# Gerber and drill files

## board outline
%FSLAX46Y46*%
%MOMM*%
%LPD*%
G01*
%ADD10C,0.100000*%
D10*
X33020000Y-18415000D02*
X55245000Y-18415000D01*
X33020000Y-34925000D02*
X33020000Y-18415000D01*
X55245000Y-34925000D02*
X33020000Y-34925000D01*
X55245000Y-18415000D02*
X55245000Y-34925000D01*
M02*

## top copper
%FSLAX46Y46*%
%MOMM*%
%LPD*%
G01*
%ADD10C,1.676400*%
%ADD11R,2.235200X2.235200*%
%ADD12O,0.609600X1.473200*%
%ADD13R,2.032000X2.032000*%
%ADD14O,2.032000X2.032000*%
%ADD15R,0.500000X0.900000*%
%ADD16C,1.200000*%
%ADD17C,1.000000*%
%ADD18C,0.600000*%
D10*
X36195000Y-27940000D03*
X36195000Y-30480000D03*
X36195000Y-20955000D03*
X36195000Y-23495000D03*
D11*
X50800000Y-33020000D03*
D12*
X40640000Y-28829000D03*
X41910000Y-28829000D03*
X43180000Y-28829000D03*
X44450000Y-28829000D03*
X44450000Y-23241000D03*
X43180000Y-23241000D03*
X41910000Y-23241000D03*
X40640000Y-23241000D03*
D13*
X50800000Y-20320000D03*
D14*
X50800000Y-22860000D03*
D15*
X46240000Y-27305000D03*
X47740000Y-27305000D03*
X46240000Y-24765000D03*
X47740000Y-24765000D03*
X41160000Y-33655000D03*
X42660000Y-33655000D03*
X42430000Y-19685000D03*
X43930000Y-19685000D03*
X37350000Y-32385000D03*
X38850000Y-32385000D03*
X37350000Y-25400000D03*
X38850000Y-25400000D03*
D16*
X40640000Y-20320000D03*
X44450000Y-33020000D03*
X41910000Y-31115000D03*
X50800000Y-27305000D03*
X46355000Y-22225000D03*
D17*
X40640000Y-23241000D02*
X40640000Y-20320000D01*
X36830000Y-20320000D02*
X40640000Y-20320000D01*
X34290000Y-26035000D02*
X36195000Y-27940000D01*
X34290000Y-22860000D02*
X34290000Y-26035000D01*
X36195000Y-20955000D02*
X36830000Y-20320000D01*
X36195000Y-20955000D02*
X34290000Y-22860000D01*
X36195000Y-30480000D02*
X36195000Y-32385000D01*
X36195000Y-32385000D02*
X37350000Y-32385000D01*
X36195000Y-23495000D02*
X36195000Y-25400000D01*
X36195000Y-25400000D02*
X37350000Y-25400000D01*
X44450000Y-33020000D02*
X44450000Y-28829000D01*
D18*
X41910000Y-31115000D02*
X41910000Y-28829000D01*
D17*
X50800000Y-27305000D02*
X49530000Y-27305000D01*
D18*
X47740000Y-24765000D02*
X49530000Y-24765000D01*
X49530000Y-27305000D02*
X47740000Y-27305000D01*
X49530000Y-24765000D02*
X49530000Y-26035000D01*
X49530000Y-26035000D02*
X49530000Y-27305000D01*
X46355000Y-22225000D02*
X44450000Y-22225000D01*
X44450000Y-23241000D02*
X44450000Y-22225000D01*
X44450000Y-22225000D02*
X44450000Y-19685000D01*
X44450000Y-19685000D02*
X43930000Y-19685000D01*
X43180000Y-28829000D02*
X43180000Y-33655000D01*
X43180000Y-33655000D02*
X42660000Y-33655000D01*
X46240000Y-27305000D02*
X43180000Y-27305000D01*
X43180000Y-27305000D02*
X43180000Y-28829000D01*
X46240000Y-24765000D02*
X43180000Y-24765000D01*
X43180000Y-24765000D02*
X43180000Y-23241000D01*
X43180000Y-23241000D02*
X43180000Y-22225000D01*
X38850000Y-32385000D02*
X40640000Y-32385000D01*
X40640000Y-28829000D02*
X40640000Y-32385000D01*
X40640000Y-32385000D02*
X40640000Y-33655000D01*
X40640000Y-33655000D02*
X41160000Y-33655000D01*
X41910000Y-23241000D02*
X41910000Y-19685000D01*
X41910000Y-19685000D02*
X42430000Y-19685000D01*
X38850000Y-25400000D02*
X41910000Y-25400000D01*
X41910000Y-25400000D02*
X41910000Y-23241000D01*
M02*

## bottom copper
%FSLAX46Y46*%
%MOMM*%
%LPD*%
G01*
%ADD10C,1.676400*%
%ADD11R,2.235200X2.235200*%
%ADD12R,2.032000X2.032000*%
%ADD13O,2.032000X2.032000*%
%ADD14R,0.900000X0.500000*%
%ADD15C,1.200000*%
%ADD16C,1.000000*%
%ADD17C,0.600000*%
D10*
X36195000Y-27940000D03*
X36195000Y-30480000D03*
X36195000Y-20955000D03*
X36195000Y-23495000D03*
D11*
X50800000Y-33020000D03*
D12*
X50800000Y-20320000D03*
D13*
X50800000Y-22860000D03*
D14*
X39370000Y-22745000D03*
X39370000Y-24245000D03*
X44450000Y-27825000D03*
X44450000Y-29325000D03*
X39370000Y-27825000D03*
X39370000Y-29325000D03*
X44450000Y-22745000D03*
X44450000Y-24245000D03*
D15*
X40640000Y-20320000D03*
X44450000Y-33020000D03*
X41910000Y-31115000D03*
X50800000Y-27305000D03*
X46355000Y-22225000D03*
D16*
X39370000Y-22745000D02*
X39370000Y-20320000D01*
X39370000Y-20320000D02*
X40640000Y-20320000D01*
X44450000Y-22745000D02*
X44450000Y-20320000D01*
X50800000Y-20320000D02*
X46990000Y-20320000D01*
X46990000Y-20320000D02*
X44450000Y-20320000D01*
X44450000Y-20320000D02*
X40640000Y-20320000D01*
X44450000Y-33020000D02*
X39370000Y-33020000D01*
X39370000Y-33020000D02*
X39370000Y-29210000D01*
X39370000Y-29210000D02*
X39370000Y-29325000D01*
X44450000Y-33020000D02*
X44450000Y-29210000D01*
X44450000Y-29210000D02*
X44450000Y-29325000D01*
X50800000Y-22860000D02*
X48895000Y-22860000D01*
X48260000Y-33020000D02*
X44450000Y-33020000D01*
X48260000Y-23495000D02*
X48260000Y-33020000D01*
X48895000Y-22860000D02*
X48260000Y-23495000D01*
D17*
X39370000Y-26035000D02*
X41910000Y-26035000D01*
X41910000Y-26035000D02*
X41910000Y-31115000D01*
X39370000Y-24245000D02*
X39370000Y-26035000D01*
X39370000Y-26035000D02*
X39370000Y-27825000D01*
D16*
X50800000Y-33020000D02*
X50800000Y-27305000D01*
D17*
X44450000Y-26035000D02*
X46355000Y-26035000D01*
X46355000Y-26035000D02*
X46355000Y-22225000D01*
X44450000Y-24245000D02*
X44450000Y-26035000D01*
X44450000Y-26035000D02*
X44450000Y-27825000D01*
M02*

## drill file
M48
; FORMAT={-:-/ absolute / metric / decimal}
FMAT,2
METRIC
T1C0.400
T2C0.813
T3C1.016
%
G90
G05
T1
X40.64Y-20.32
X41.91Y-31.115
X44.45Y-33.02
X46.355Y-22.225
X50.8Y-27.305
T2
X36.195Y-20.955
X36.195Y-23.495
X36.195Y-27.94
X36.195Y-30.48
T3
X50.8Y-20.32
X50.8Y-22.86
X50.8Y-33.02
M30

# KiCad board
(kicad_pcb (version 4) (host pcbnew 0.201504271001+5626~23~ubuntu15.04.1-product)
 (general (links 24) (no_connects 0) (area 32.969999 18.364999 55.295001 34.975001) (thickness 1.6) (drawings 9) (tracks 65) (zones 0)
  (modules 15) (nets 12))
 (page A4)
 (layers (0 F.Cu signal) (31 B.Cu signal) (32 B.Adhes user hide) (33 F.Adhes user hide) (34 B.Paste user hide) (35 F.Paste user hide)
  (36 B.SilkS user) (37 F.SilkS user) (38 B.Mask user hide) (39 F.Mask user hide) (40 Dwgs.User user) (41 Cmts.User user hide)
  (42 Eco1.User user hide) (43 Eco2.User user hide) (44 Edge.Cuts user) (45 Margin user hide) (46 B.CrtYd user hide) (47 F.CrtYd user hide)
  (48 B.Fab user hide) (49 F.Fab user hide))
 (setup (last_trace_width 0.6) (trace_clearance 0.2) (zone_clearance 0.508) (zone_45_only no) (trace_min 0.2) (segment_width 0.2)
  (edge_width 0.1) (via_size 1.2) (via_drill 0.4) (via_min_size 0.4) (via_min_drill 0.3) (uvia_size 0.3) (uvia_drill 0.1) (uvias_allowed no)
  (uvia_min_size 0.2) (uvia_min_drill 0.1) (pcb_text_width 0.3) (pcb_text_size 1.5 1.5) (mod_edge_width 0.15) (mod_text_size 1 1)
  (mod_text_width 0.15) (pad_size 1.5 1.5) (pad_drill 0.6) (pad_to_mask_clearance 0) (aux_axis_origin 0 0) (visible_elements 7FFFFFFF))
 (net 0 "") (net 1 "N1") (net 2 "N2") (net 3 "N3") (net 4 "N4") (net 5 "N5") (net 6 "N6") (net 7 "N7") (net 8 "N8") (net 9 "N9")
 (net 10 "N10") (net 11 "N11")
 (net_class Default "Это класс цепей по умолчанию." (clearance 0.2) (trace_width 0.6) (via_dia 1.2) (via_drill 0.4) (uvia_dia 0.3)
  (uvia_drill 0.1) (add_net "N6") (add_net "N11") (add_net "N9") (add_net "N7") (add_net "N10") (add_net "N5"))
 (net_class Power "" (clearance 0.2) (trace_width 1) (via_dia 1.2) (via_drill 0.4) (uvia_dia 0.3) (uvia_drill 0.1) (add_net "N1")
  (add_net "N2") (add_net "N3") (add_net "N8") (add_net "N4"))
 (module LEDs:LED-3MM (layer B.Cu) (at 36.195 29.21 270)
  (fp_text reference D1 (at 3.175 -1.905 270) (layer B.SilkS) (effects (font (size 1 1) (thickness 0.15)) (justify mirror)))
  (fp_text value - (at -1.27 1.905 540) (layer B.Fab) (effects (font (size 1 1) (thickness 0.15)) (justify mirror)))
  (pad 1 thru_hole circle (at -1.27 0 270) (size 1.6764 1.6764) (drill 0.8128) (layers *.Cu *.Mask B.SilkS) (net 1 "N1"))
  (pad 2 thru_hole circle (at 1.27 0 270) (size 1.6764 1.6764) (drill 0.8128) (layers *.Cu *.Mask B.SilkS) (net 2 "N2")))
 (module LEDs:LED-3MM (layer B.Cu) (at 36.195 22.225 270)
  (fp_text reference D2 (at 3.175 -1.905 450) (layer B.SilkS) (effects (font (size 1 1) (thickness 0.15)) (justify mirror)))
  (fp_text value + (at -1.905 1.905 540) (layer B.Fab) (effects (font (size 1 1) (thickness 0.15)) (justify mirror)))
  (pad 1 thru_hole circle (at -1.27 0 270) (size 1.6764 1.6764) (drill 0.8128) (layers *.Cu *.Mask B.SilkS) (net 1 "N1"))
  (pad 2 thru_hole circle (at 1.27 0 270) (size 1.6764 1.6764) (drill 0.8128) (layers *.Cu *.Mask B.SilkS) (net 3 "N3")))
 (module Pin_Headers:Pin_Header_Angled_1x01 (layer F.Cu) (at 50.8 33.02)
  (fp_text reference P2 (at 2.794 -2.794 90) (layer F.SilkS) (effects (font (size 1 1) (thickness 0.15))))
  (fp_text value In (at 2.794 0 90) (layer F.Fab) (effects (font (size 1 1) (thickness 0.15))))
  (pad 1 thru_hole rect (at 0 0) (size 2.2352 2.2352) (drill 1.016) (layers *.Cu *.Mask F.SilkS) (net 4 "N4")))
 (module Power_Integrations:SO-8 (layer F.Cu) (at 42.545 26.035)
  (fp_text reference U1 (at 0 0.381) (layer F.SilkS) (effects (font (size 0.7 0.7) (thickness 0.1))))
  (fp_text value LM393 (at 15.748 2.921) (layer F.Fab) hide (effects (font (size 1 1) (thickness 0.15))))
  (pad 1 smd oval (at -1.905 2.794) (size 0.6096 1.4732) (layers F.Cu F.Paste F.Mask) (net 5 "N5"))
  (pad 2 smd oval (at -0.635 2.794) (size 0.6096 1.4732) (layers F.Cu F.Paste F.Mask) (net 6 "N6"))
  (pad 3 smd oval (at 0.635 2.794) (size 0.6096 1.4732) (layers F.Cu F.Paste F.Mask) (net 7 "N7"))
  (pad 4 smd oval (at 1.905 2.794) (size 0.6096 1.4732) (layers F.Cu F.Paste F.Mask) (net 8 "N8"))
  (pad 5 smd oval (at 1.905 -2.794) (size 0.6096 1.4732) (layers F.Cu F.Paste F.Mask) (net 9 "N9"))
  (pad 6 smd oval (at 0.635 -2.794) (size 0.6096 1.4732) (layers F.Cu F.Paste F.Mask) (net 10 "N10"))
  (pad 7 smd oval (at -0.635 -2.794) (size 0.6096 1.4732) (layers F.Cu F.Paste F.Mask) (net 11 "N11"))
  (pad 8 smd oval (at -1.905 -2.794) (size 0.6096 1.4732) (layers F.Cu F.Paste F.Mask) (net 1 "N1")))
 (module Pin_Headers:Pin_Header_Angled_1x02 (layer F.Cu) (at 50.8 20.32)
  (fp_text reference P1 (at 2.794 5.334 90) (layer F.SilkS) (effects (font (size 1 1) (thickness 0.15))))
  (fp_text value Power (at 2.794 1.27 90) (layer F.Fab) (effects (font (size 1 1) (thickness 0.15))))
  (pad 1 thru_hole rect (at 0 0) (size 2.032 2.032) (drill 1.016) (layers *.Cu *.Mask F.SilkS) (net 1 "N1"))
  (pad 2 thru_hole oval (at 0 2.54) (size 2.032 2.032) (drill 1.016) (layers *.Cu *.Mask F.SilkS) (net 8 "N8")))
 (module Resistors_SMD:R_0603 (layer B.Cu) (at 39.37 23.495 270)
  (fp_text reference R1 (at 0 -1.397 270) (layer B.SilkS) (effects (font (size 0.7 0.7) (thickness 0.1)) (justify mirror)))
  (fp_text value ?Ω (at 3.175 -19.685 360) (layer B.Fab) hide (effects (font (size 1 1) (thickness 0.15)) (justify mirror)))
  (pad 1 smd rect (at -0.75 0 270) (size 0.5 0.9) (layers B.Cu B.Paste B.Mask) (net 1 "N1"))
  (pad 2 smd rect (at 0.75 0 270) (size 0.5 0.9) (layers B.Cu B.Paste B.Mask) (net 6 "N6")))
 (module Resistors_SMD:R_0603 (layer B.Cu) (at 44.45 28.575 270)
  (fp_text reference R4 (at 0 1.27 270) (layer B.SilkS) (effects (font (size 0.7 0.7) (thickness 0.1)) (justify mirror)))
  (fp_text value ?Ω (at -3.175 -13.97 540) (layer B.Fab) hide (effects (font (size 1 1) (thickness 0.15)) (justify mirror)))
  (pad 1 smd rect (at -0.75 0 270) (size 0.5 0.9) (layers B.Cu B.Paste B.Mask) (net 9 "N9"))
  (pad 2 smd rect (at 0.75 0 270) (size 0.5 0.9) (layers B.Cu B.Paste B.Mask) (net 8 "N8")))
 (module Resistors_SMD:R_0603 (layer B.Cu) (at 39.37 28.575 270)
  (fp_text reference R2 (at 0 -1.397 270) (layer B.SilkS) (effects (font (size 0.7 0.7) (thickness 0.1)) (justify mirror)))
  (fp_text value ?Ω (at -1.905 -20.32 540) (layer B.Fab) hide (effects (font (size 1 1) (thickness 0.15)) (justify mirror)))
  (pad 1 smd rect (at -0.75 0 270) (size 0.5 0.9) (layers B.Cu B.Paste B.Mask) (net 6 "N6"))
  (pad 2 smd rect (at 0.75 0 270) (size 0.5 0.9) (layers B.Cu B.Paste B.Mask) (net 8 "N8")))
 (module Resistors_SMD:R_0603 (layer B.Cu) (at 44.45 23.495 270)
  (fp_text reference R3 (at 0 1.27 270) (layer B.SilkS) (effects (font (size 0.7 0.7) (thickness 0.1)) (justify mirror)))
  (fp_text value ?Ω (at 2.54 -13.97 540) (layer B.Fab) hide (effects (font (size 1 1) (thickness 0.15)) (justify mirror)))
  (pad 1 smd rect (at -0.75 0 270) (size 0.5 0.9) (layers B.Cu B.Paste B.Mask) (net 1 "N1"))
  (pad 2 smd rect (at 0.75 0 270) (size 0.5 0.9) (layers B.Cu B.Paste B.Mask) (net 9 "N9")))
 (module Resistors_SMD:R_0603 (layer F.Cu) (at 46.99 27.305)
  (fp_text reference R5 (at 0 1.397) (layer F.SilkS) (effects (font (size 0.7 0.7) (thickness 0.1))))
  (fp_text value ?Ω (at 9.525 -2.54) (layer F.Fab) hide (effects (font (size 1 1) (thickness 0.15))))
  (pad 1 smd rect (at -0.75 0) (size 0.5 0.9) (layers F.Cu F.Paste F.Mask) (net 7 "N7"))
  (pad 2 smd rect (at 0.75 0) (size 0.5 0.9) (layers F.Cu F.Paste F.Mask) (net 4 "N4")))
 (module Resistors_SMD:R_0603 (layer F.Cu) (at 46.99 24.765)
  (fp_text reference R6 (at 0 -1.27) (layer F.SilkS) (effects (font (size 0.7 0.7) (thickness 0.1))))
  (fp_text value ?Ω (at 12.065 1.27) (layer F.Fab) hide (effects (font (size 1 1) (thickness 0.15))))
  (pad 1 smd rect (at -0.75 0) (size 0.5 0.9) (layers F.Cu F.Paste F.Mask) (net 10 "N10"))
  (pad 2 smd rect (at 0.75 0) (size 0.5 0.9) (layers F.Cu F.Paste F.Mask) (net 4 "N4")))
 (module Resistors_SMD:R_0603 (layer F.Cu) (at 41.91 33.655)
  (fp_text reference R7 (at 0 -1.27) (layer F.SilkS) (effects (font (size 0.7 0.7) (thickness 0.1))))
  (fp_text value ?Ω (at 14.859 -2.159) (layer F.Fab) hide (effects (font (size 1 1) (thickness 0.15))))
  (pad 1 smd rect (at -0.75 0) (size 0.5 0.9) (layers F.Cu F.Paste F.Mask) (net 5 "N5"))
  (pad 2 smd rect (at 0.75 0) (size 0.5 0.9) (layers F.Cu F.Paste F.Mask) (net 7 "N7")))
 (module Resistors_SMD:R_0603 (layer F.Cu) (at 43.18 19.685)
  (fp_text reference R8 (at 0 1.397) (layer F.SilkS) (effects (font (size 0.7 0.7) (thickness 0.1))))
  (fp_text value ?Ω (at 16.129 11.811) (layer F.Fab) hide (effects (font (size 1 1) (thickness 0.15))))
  (pad 1 smd rect (at -0.75 0) (size 0.5 0.9) (layers F.Cu F.Paste F.Mask) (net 11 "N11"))
  (pad 2 smd rect (at 0.75 0) (size 0.5 0.9) (layers F.Cu F.Paste F.Mask) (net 9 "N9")))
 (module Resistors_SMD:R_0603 (layer F.Cu) (at 38.1 32.385)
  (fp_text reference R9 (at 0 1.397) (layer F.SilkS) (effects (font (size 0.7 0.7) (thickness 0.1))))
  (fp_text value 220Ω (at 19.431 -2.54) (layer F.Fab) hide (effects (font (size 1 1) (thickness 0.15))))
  (pad 1 smd rect (at -0.75 0) (size 0.5 0.9) (layers F.Cu F.Paste F.Mask) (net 2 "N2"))
  (pad 2 smd rect (at 0.75 0) (size 0.5 0.9) (layers F.Cu F.Paste F.Mask) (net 5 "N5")))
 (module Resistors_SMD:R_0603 (layer F.Cu) (at 38.1 25.4)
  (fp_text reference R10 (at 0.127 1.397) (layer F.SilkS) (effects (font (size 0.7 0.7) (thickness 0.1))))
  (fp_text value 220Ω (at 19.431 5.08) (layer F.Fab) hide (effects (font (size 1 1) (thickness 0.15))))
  (pad 1 smd rect (at -0.75 0) (size 0.5 0.9) (layers F.Cu F.Paste F.Mask) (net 3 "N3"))
  (pad 2 smd rect (at 0.75 0) (size 0.5 0.9) (layers F.Cu F.Paste F.Mask) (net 11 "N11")))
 (gr_line (start 33.02 18.415) (end 55.245 18.415) (angle 90) (layer Edge.Cuts) (width 0.1))
 (gr_line (start 33.02 34.925) (end 33.02 18.415) (angle 90) (layer Edge.Cuts) (width 0.1))
 (gr_line (start 55.245 34.925) (end 33.02 34.925) (angle 90) (layer Edge.Cuts) (width 0.1))
 (gr_line (start 55.245 18.415) (end 55.245 34.925) (angle 90) (layer Edge.Cuts) (width 0.1))
 (segment (start 39.37 22.745) (end 39.37 20.32) (width 1) (layer B.Cu) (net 1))
 (segment (start 39.37 20.32) (end 40.64 20.32) (width 1) (layer B.Cu) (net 1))
 (segment (start 44.45 22.745) (end 44.45 20.32) (width 1) (layer B.Cu) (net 1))
 (segment (start 50.8 20.32) (end 46.99 20.32) (width 1) (layer B.Cu) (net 1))
 (segment (start 46.99 20.32) (end 44.45 20.32) (width 1) (layer B.Cu) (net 1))
 (segment (start 44.45 20.32) (end 40.64 20.32) (width 1) (layer B.Cu) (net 1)) (via (at 40.64 20.32) (size 1.2) (layers F.Cu B.Cu) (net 1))
 (segment (start 40.64 23.241) (end 40.64 20.32) (width 1) (layer F.Cu) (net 1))
 (segment (start 36.83 20.32) (end 40.64 20.32) (width 1) (layer F.Cu) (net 1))
 (segment (start 34.29 26.035) (end 36.195 27.94) (width 1) (layer F.Cu) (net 1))
 (segment (start 34.29 22.86) (end 34.29 26.035) (width 1) (layer F.Cu) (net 1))
 (segment (start 36.195 20.955) (end 36.83 20.32) (width 1) (layer F.Cu) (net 1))
 (segment (start 36.195 20.955) (end 34.29 22.86) (width 1) (layer F.Cu) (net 1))
 (segment (start 36.195 30.48) (end 36.195 32.385) (width 1) (layer F.Cu) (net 2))
 (segment (start 36.195 32.385) (end 37.35 32.385) (width 1) (layer F.Cu) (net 2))
 (segment (start 36.195 23.495) (end 36.195 25.4) (width 1) (layer F.Cu) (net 3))
 (segment (start 36.195 25.4) (end 37.35 25.4) (width 1) (layer F.Cu) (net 3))
 (segment (start 44.45 33.02) (end 39.37 33.02) (width 1) (layer B.Cu) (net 8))
 (segment (start 39.37 33.02) (end 39.37 29.21) (width 1) (layer B.Cu) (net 8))
 (segment (start 39.37 29.21) (end 39.37 29.325) (width 1) (layer B.Cu) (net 8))
 (segment (start 44.45 33.02) (end 44.45 29.21) (width 1) (layer B.Cu) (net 8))
 (segment (start 44.45 29.21) (end 44.45 29.325) (width 1) (layer B.Cu) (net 8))
 (segment (start 50.8 22.86) (end 48.895 22.86) (width 1) (layer B.Cu) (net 8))
 (segment (start 44.45 33.02) (end 44.45 28.829) (width 1) (layer F.Cu) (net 8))
 (via (at 44.45 33.02) (size 1.2) (layers F.Cu B.Cu) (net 8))
 (segment (start 48.26 33.02) (end 44.45 33.02) (width 1) (layer B.Cu) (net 8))
 (segment (start 48.26 23.495) (end 48.26 33.02) (width 1) (layer B.Cu) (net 8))
 (segment (start 48.895 22.86) (end 48.26 23.495) (width 1) (layer B.Cu) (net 8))
 (segment (start 39.37 26.035) (end 41.91 26.035) (width 0.6) (layer B.Cu) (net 6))
 (segment (start 41.91 31.115) (end 41.91 28.829) (width 0.6) (layer F.Cu) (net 6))
 (via (at 41.91 31.115) (size 1.2) (layers F.Cu B.Cu) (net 6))
 (segment (start 41.91 26.035) (end 41.91 31.115) (width 0.6) (layer B.Cu) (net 6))
 (segment (start 39.37 24.245) (end 39.37 26.035) (width 0.6) (layer B.Cu) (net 6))
 (segment (start 39.37 26.035) (end 39.37 27.825) (width 0.6) (layer B.Cu) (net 6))
 (segment (start 50.8 33.02) (end 50.8 27.305) (width 1) (layer B.Cu) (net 4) (status 400000))
 (segment (start 50.8 27.305) (end 49.53 27.305) (width 1) (layer F.Cu) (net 4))
 (via (at 50.8 27.305) (size 1.2) (layers F.Cu B.Cu) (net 4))
 (segment (start 47.74 24.765) (end 49.53 24.765) (width 0.6) (layer F.Cu) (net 4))
 (segment (start 49.53 27.305) (end 47.74 27.305) (width 0.6) (layer F.Cu) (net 4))
 (segment (start 49.53 24.765) (end 49.53 26.035) (width 0.6) (layer F.Cu) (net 4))
 (segment (start 49.53 26.035) (end 49.53 27.305) (width 0.6) (layer F.Cu) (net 4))
 (segment (start 44.45 26.035) (end 46.355 26.035) (width 0.6) (layer B.Cu) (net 9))
 (segment (start 46.355 22.225) (end 44.45 22.225) (width 0.6) (layer F.Cu) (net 9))
 (via (at 46.355 22.225) (size 1.2) (layers F.Cu B.Cu) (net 9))
 (segment (start 46.355 26.035) (end 46.355 22.225) (width 0.6) (layer B.Cu) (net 9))
 (segment (start 44.45 24.245) (end 44.45 26.035) (width 0.6) (layer B.Cu) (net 9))
 (segment (start 44.45 26.035) (end 44.45 27.825) (width 0.6) (layer B.Cu) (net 9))
 (segment (start 44.45 23.241) (end 44.45 22.225) (width 0.6) (layer F.Cu) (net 9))
 (segment (start 44.45 22.225) (end 44.45 19.685) (width 0.6) (layer F.Cu) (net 9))
 (segment (start 44.45 19.685) (end 43.93 19.685) (width 0.6) (layer F.Cu) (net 9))
 (segment (start 43.18 28.829) (end 43.18 33.655) (width 0.6) (layer F.Cu) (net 7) (status 400000))
 (segment (start 43.18 33.655) (end 42.66 33.655) (width 0.6) (layer F.Cu) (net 7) (status 800000))
 (segment (start 46.24 27.305) (end 43.18 27.305) (width 0.6) (layer F.Cu) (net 7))
 (segment (start 43.18 27.305) (end 43.18 28.829) (width 0.6) (layer F.Cu) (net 7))
 (segment (start 46.24 24.765) (end 43.18 24.765) (width 0.6) (layer F.Cu) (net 10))
 (segment (start 43.18 24.765) (end 43.18 23.241) (width 0.6) (layer F.Cu) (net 10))
 (segment (start 43.18 23.241) (end 43.18 22.225) (width 0.6) (layer F.Cu) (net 10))
 (segment (start 38.85 32.385) (end 40.64 32.385) (width 0.6) (layer F.Cu) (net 5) (status 400000))
 (segment (start 40.64 28.829) (end 40.64 32.385) (width 0.6) (layer F.Cu) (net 5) (status 400000))
 (segment (start 40.64 32.385) (end 40.64 33.655) (width 0.6) (layer F.Cu) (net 5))
 (segment (start 40.64 33.655) (end 41.16 33.655) (width 0.6) (layer F.Cu) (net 5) (status 800000))
 (segment (start 41.91 23.241) (end 41.91 19.685) (width 0.6) (layer F.Cu) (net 11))
 (segment (start 41.91 19.685) (end 42.43 19.685) (width 0.6) (layer F.Cu) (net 11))
 (segment (start 38.85 25.4) (end 41.91 25.4) (width 0.6) (layer F.Cu) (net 11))
 (segment (start 41.91 25.4) (end 41.91 23.241) (width 0.6) (layer F.Cu) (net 11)))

